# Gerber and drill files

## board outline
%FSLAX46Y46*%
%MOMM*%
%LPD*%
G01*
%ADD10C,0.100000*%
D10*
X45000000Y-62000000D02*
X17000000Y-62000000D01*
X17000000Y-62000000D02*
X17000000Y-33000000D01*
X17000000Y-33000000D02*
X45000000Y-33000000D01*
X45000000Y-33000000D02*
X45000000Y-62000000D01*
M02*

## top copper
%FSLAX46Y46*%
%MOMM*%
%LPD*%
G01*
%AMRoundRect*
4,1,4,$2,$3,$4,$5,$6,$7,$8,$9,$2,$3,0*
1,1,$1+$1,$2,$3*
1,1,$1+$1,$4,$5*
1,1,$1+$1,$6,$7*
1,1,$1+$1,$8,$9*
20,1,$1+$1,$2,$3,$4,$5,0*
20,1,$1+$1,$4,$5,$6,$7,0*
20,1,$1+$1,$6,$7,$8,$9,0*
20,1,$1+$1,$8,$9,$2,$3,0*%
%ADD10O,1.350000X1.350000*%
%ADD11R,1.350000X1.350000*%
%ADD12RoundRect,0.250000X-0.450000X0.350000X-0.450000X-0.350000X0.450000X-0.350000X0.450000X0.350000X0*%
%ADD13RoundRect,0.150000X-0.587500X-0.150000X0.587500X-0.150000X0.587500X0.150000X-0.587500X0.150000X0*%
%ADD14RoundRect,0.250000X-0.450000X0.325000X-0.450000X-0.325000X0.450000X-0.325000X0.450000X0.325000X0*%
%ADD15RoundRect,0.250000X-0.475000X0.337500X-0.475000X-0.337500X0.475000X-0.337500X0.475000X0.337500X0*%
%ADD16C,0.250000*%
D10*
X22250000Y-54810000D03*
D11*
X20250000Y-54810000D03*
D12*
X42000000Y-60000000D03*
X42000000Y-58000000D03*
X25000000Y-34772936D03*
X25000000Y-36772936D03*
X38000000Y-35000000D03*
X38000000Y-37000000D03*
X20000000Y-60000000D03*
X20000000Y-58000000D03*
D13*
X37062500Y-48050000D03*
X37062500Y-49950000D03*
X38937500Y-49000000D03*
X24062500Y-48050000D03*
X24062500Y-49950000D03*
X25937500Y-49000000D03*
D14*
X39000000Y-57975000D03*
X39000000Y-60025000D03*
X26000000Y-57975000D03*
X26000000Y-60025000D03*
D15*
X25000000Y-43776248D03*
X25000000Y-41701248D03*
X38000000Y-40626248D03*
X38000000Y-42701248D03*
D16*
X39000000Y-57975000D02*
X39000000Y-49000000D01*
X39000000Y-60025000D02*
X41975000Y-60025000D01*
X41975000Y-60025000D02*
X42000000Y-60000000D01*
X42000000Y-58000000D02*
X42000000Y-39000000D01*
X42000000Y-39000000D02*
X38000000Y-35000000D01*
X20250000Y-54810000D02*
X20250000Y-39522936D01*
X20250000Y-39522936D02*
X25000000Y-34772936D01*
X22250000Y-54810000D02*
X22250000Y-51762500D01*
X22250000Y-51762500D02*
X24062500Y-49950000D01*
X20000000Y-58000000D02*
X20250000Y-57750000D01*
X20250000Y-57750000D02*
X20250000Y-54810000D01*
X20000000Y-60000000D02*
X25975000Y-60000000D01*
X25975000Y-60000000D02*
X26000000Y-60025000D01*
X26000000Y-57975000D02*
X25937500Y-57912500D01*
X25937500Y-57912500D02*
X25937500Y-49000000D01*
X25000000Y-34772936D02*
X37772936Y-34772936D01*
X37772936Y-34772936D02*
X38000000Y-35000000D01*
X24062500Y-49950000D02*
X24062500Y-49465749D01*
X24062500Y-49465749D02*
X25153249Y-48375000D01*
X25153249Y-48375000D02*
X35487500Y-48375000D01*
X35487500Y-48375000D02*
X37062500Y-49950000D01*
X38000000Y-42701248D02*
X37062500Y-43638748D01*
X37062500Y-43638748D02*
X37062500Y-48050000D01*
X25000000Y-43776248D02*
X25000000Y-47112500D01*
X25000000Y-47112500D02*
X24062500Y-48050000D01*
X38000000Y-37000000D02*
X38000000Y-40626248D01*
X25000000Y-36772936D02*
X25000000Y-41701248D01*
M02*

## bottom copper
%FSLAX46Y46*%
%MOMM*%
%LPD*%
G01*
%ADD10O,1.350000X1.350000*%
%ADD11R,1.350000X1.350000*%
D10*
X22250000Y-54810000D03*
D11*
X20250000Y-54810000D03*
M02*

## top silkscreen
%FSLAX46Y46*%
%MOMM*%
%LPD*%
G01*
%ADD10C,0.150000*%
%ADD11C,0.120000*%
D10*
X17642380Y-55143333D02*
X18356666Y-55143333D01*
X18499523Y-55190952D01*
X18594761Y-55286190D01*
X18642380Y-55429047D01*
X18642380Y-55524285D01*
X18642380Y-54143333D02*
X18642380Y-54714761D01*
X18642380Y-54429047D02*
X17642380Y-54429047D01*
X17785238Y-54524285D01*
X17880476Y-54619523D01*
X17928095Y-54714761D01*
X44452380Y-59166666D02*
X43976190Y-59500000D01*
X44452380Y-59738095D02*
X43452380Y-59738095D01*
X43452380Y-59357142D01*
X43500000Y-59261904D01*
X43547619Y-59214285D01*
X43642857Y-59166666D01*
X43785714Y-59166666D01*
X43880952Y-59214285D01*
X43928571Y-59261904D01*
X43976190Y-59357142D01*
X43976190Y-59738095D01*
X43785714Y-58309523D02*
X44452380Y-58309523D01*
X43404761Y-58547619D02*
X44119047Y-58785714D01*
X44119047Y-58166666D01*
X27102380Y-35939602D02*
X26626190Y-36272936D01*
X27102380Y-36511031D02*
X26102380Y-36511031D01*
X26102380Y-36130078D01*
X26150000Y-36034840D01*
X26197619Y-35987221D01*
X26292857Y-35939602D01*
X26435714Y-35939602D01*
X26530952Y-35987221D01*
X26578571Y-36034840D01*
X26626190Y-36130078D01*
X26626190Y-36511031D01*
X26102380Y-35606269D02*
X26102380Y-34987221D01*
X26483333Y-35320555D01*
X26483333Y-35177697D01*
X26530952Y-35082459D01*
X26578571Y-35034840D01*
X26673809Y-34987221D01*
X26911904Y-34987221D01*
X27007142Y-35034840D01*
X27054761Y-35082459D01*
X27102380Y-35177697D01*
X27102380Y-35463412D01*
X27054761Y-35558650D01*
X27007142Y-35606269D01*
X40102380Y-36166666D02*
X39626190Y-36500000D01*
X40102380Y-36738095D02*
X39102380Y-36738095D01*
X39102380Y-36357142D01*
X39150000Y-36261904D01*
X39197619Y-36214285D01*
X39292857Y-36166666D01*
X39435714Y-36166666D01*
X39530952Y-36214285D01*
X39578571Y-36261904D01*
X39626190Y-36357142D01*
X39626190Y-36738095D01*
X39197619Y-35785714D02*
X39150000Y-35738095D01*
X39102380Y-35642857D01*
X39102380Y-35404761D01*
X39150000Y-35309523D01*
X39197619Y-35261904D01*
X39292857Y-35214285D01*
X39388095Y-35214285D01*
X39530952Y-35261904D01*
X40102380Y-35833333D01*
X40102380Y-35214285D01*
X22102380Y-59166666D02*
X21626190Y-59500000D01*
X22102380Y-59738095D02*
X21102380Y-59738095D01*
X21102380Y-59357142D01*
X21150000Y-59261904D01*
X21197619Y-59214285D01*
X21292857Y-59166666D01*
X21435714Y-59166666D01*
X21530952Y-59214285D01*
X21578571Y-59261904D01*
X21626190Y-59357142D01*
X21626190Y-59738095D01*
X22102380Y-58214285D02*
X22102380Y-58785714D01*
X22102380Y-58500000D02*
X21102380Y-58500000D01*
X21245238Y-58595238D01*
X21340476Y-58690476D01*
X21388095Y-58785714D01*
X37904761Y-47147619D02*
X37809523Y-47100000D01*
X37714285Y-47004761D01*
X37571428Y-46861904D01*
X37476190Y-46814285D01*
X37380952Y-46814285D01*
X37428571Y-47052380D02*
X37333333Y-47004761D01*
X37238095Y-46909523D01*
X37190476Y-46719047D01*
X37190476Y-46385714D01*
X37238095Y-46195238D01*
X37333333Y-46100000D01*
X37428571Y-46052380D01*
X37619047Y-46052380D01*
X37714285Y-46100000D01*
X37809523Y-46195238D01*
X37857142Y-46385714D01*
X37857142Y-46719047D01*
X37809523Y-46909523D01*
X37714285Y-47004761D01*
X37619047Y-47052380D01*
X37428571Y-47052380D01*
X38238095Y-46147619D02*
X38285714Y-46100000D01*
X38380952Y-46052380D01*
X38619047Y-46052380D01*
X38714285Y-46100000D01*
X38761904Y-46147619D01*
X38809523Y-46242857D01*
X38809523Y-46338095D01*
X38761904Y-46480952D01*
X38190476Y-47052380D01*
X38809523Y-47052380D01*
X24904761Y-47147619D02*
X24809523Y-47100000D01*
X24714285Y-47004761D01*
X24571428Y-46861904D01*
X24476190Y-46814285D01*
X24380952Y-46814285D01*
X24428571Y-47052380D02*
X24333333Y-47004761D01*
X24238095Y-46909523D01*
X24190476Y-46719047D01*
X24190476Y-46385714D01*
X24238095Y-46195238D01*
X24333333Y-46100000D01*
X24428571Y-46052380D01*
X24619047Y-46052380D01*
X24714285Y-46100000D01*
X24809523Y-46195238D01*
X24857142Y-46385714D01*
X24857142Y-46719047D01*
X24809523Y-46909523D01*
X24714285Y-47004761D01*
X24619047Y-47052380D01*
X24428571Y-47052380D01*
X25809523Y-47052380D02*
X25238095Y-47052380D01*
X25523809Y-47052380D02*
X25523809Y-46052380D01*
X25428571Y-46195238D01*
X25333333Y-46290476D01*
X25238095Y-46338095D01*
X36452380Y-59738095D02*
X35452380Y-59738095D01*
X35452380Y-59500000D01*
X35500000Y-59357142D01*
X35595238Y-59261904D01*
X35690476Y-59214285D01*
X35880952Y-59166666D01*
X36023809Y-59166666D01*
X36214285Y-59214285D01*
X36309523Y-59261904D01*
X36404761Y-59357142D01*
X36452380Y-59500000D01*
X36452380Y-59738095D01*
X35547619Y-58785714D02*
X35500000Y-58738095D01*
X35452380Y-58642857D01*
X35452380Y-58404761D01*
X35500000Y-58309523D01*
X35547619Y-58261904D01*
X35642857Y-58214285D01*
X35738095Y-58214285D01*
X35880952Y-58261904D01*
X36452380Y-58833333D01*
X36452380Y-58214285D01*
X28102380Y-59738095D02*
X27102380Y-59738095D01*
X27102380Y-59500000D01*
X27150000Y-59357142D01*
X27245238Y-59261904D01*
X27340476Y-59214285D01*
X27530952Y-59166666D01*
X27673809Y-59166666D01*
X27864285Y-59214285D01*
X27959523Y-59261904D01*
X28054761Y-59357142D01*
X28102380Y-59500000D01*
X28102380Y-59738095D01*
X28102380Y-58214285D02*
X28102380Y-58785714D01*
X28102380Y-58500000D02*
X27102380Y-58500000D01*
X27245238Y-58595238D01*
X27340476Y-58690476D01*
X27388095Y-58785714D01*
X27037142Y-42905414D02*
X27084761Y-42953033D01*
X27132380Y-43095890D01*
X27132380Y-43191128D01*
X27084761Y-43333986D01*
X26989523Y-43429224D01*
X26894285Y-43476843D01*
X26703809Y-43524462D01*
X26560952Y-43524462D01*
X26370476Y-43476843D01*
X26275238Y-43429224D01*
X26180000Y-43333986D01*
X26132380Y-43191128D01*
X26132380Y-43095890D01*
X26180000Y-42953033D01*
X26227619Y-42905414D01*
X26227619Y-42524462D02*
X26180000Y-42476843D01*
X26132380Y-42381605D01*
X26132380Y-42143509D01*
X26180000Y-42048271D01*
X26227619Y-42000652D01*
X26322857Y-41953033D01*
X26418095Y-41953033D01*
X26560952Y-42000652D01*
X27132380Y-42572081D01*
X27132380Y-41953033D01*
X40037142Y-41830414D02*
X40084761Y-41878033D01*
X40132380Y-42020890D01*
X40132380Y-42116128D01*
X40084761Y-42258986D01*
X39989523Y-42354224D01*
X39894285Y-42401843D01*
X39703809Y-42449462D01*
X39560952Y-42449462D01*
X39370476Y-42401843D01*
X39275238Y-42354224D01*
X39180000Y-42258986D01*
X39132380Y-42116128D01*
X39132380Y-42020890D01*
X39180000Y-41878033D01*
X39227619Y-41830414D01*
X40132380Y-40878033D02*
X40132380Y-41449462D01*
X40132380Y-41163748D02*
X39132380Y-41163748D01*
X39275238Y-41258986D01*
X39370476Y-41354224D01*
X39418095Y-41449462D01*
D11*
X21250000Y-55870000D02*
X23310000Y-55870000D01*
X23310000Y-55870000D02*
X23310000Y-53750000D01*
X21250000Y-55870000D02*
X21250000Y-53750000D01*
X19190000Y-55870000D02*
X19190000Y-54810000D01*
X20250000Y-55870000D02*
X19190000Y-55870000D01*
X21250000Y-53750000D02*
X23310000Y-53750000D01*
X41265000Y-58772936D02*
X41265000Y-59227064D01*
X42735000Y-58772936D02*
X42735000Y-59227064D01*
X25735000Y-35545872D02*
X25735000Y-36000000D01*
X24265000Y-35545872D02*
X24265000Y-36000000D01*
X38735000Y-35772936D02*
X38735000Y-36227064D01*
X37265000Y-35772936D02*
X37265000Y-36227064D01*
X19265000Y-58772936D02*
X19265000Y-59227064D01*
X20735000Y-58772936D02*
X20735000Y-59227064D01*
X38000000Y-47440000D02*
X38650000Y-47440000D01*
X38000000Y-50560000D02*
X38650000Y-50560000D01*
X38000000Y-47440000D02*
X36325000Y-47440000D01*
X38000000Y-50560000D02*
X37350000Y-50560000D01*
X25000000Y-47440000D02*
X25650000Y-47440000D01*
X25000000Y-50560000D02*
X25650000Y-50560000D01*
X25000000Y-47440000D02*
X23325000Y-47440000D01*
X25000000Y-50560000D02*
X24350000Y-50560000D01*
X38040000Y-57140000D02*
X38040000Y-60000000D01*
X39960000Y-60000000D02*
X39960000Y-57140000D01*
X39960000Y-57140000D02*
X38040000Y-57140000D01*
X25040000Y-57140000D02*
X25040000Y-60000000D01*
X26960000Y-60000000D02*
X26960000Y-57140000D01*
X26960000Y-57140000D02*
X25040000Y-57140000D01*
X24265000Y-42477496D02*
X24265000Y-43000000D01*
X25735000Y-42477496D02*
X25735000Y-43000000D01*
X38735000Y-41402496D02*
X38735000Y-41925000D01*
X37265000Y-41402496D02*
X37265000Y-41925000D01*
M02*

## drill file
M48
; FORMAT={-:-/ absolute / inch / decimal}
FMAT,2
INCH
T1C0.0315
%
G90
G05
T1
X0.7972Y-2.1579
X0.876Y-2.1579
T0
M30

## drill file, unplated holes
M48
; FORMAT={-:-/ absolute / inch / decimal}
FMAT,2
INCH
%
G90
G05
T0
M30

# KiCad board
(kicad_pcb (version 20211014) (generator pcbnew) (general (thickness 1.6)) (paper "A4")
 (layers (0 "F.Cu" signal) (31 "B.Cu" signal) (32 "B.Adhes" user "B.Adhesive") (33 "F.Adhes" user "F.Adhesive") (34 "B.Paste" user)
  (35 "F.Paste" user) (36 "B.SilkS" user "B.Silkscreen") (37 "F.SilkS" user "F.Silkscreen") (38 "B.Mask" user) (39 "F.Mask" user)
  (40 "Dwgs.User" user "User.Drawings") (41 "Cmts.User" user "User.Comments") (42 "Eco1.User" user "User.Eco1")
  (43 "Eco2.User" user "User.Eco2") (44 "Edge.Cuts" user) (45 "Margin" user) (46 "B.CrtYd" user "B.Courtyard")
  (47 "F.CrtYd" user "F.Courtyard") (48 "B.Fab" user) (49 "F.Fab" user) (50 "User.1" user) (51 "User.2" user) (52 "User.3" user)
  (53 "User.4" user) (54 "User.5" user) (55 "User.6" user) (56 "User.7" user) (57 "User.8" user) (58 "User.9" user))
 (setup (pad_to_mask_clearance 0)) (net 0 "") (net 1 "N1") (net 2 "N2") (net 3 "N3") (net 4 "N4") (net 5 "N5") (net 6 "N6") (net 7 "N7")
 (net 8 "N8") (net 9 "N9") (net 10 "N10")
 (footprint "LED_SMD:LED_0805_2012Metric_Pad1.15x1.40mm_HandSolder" (layer "F.Cu") (at 26 59 -90)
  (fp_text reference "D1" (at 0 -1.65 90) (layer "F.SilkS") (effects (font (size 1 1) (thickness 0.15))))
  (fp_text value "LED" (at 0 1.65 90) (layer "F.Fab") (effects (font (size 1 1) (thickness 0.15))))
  (fp_line (start 1 -0.96) (end -1.86 -0.96) (layer "F.SilkS") (width 0.12))
  (fp_line (start -1.86 -0.96) (end -1.86 0.96) (layer "F.SilkS") (width 0.12))
  (fp_line (start -1.86 0.96) (end 1 0.96) (layer "F.SilkS") (width 0.12))
  (pad "1" smd roundrect (at -1.025 0 270) (size 1.15 1.4) (layers "F.Cu" "F.Paste" "F.Mask") (roundrect_rratio 0.2173913043) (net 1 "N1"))
  (pad "2" smd roundrect (at 1.025 0 270) (size 1.15 1.4) (layers "F.Cu" "F.Paste" "F.Mask") (roundrect_rratio 0.2173913043) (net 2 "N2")))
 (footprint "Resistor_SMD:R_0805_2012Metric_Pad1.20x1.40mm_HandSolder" (layer "F.Cu") (at 25 35.772936 -90)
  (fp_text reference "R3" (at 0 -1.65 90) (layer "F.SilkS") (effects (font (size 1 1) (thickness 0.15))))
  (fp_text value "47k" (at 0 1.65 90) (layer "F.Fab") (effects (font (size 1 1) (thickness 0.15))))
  (fp_line (start -0.227064 0.735) (end 0.227064 0.735) (layer "F.SilkS") (width 0.12))
  (fp_line (start -0.227064 -0.735) (end 0.227064 -0.735) (layer "F.SilkS") (width 0.12))
  (pad "1" smd roundrect (at -1 0 270) (size 1.2 1.4) (layers "F.Cu" "F.Paste" "F.Mask") (roundrect_rratio 0.2083333333) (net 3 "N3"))
  (pad "2" smd roundrect (at 1 0 270) (size 1.2 1.4) (layers "F.Cu" "F.Paste" "F.Mask") (roundrect_rratio 0.2083333333) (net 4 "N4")))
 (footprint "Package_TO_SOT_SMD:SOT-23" (layer "F.Cu") (at 38 49)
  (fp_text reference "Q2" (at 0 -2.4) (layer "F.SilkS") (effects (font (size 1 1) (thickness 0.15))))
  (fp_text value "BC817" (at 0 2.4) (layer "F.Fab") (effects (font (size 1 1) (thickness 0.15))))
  (fp_line (start 0 -1.56) (end -1.675 -1.56) (layer "F.SilkS") (width 0.12))
  (fp_line (start 0 1.56) (end -0.65 1.56) (layer "F.SilkS") (width 0.12))
  (fp_line (start 0 1.56) (end 0.65 1.56) (layer "F.SilkS") (width 0.12))
  (fp_line (start 0 -1.56) (end 0.65 -1.56) (layer "F.SilkS") (width 0.12))
  (pad "1" smd roundrect (at -0.9375 -0.95) (size 1.475 0.6) (layers "F.Cu" "F.Paste" "F.Mask") (roundrect_rratio 0.25) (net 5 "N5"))
  (pad "2" smd roundrect (at -0.9375 0.95) (size 1.475 0.6) (layers "F.Cu" "F.Paste" "F.Mask") (roundrect_rratio 0.25) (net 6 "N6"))
  (pad "3" smd roundrect (at 0.9375 0) (size 1.475 0.6) (layers "F.Cu" "F.Paste" "F.Mask") (roundrect_rratio 0.25) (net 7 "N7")))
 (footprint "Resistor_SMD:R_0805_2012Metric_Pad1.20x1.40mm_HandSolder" (layer "F.Cu") (at 38 36 -90)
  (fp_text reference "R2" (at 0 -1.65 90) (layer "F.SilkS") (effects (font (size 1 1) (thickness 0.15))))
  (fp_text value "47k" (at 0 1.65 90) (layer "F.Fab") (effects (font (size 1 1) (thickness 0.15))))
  (fp_line (start -0.227064 -0.735) (end 0.227064 -0.735) (layer "F.SilkS") (width 0.12))
  (fp_line (start -0.227064 0.735) (end 0.227064 0.735) (layer "F.SilkS") (width 0.12))
  (pad "1" smd roundrect (at -1 0 270) (size 1.2 1.4) (layers "F.Cu" "F.Paste" "F.Mask") (roundrect_rratio 0.2083333333) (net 3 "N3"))
  (pad "2" smd roundrect (at 1 0 270) (size 1.2 1.4) (layers "F.Cu" "F.Paste" "F.Mask") (roundrect_rratio 0.2083333333) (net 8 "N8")))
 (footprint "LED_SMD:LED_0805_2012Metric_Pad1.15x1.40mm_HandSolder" (layer "F.Cu") (at 39 59 -90)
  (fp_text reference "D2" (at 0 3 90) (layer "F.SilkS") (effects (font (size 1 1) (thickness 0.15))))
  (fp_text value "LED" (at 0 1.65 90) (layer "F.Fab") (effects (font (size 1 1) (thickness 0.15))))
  (fp_line (start -1.86 -0.96) (end -1.86 0.96) (layer "F.SilkS") (width 0.12))
  (fp_line (start -1.86 0.96) (end 1 0.96) (layer "F.SilkS") (width 0.12))
  (fp_line (start 1 -0.96) (end -1.86 -0.96) (layer "F.SilkS") (width 0.12))
  (pad "1" smd roundrect (at -1.025 0 270) (size 1.15 1.4) (layers "F.Cu" "F.Paste" "F.Mask") (roundrect_rratio 0.2173913043) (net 7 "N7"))
  (pad "2" smd roundrect (at 1.025 0 270) (size 1.15 1.4) (layers "F.Cu" "F.Paste" "F.Mask") (roundrect_rratio 0.2173913043) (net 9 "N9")))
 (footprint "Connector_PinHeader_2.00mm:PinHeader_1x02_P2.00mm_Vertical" (layer "F.Cu") (at 20.25 54.81 90)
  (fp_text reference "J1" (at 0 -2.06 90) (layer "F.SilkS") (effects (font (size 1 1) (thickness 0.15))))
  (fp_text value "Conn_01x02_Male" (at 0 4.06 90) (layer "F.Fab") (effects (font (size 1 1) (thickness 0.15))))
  (fp_line (start -1.06 0) (end -1.06 -1.06) (layer "F.SilkS") (width 0.12))
  (fp_line (start -1.06 -1.06) (end 0 -1.06) (layer "F.SilkS") (width 0.12))
  (fp_line (start -1.06 1) (end 1.06 1) (layer "F.SilkS") (width 0.12))
  (fp_line (start -1.06 1) (end -1.06 3.06) (layer "F.SilkS") (width 0.12))
  (fp_line (start 1.06 1) (end 1.06 3.06) (layer "F.SilkS") (width 0.12))
  (fp_line (start -1.06 3.06) (end 1.06 3.06) (layer "F.SilkS") (width 0.12))
  (pad "1" thru_hole rect (at 0 0 90) (size 1.35 1.35) (drill 0.8) (layers *.Cu *.Mask) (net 3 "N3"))
  (pad "2" thru_hole oval (at 0 2 90) (size 1.35 1.35) (drill 0.8) (layers *.Cu *.Mask) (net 6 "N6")))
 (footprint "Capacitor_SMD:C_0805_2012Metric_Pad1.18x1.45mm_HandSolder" (layer "F.Cu") (at 38 41.663748 -90)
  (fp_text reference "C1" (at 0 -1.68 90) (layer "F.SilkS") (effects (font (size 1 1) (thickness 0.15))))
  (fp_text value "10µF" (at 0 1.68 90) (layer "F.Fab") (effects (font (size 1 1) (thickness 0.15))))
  (fp_line (start -0.261252 -0.735) (end 0.261252 -0.735) (layer "F.SilkS") (width 0.12))
  (fp_line (start -0.261252 0.735) (end 0.261252 0.735) (layer "F.SilkS") (width 0.12))
  (pad "1" smd roundrect (at -1.0375 0 270) (size 1.175 1.45) (layers "F.Cu" "F.Paste" "F.Mask") (roundrect_rratio 0.2127659574)
   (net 8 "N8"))
  (pad "2" smd roundrect (at 1.0375 0 270) (size 1.175 1.45) (layers "F.Cu" "F.Paste" "F.Mask") (roundrect_rratio 0.2127659574) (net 5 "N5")))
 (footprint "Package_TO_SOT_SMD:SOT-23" (layer "F.Cu") (at 25 49)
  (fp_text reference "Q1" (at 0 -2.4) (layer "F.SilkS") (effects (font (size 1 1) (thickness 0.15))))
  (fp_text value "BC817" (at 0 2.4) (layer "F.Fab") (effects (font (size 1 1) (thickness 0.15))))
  (fp_line (start 0 -1.56) (end -1.675 -1.56) (layer "F.SilkS") (width 0.12))
  (fp_line (start 0 -1.56) (end 0.65 -1.56) (layer "F.SilkS") (width 0.12))
  (fp_line (start 0 1.56) (end -0.65 1.56) (layer "F.SilkS") (width 0.12))
  (fp_line (start 0 1.56) (end 0.65 1.56) (layer "F.SilkS") (width 0.12))
  (pad "1" smd roundrect (at -0.9375 -0.95) (size 1.475 0.6) (layers "F.Cu" "F.Paste" "F.Mask") (roundrect_rratio 0.25) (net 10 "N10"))
  (pad "2" smd roundrect (at -0.9375 0.95) (size 1.475 0.6) (layers "F.Cu" "F.Paste" "F.Mask") (roundrect_rratio 0.25) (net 6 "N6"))
  (pad "3" smd roundrect (at 0.9375 0) (size 1.475 0.6) (layers "F.Cu" "F.Paste" "F.Mask") (roundrect_rratio 0.25) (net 1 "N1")))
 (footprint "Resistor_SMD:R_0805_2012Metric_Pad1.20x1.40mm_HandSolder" (layer "F.Cu") (at 42 59 -90)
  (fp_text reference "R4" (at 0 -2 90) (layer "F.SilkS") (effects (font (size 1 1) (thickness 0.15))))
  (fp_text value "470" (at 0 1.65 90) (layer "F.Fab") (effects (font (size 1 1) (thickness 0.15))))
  (fp_line (start -0.227064 -0.735) (end 0.227064 -0.735) (layer "F.SilkS") (width 0.12))
  (fp_line (start -0.227064 0.735) (end 0.227064 0.735) (layer "F.SilkS") (width 0.12))
  (pad "1" smd roundrect (at -1 0 270) (size 1.2 1.4) (layers "F.Cu" "F.Paste" "F.Mask") (roundrect_rratio 0.2083333333) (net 3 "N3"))
  (pad "2" smd roundrect (at 1 0 270) (size 1.2 1.4) (layers "F.Cu" "F.Paste" "F.Mask") (roundrect_rratio 0.2083333333) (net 9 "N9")))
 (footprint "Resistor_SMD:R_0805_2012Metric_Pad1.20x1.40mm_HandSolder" (layer "F.Cu") (at 20 59 -90)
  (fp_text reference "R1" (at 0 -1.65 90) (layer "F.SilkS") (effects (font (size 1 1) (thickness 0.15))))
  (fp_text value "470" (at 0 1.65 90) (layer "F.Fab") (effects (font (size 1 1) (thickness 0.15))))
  (fp_line (start -0.227064 0.735) (end 0.227064 0.735) (layer "F.SilkS") (width 0.12))
  (fp_line (start -0.227064 -0.735) (end 0.227064 -0.735) (layer "F.SilkS") (width 0.12))
  (pad "1" smd roundrect (at -1 0 270) (size 1.2 1.4) (layers "F.Cu" "F.Paste" "F.Mask") (roundrect_rratio 0.2083333333) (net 3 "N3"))
  (pad "2" smd roundrect (at 1 0 270) (size 1.2 1.4) (layers "F.Cu" "F.Paste" "F.Mask") (roundrect_rratio 0.2083333333) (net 2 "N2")))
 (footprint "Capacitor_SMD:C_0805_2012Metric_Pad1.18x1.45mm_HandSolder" (layer "F.Cu") (at 25 42.738748 -90)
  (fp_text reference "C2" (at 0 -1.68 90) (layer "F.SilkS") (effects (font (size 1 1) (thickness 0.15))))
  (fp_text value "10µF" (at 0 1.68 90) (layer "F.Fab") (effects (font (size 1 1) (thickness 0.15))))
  (fp_line (start -0.261252 -0.735) (end 0.261252 -0.735) (layer "F.SilkS") (width 0.12))
  (fp_line (start -0.261252 0.735) (end 0.261252 0.735) (layer "F.SilkS") (width 0.12))
  (pad "1" smd roundrect (at -1.0375 0 270) (size 1.175 1.45) (layers "F.Cu" "F.Paste" "F.Mask") (roundrect_rratio 0.2127659574)
   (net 4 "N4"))
  (pad "2" smd roundrect (at 1.0375 0 270) (size 1.175 1.45) (layers "F.Cu" "F.Paste" "F.Mask") (roundrect_rratio 0.2127659574)
   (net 10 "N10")))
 (gr_rect (start 45 62) (end 17 33) (layer "Edge.Cuts") (width 0.1) (fill none))
 (segment (start 38 37) (end 38 40.626248) (width 0.25) (layer "F.Cu") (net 8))
 (segment (start 37.0625 43.638748) (end 37.0625 48.05) (width 0.25) (layer "F.Cu") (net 5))
 (segment (start 38 42.701248) (end 37.0625 43.638748) (width 0.25) (layer "F.Cu") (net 5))
 (segment (start 25 36.772936) (end 25 41.701248) (width 0.25) (layer "F.Cu") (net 4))
 (segment (start 25 47.1125) (end 24.0625 48.05) (width 0.25) (layer "F.Cu") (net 10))
 (segment (start 25 43.776248) (end 25 47.1125) (width 0.25) (layer "F.Cu") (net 10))
 (segment (start 26 57.975) (end 25.9375 57.9125) (width 0.25) (layer "F.Cu") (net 1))
 (segment (start 25.9375 57.9125) (end 25.9375 49) (width 0.25) (layer "F.Cu") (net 1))
 (segment (start 25.975 60) (end 26 60.025) (width 0.25) (layer "F.Cu") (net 2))
 (segment (start 20 60) (end 25.975 60) (width 0.25) (layer "F.Cu") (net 2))
 (segment (start 39 57.975) (end 39 49) (width 0.25) (layer "F.Cu") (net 7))
 (segment (start 41.975 60.025) (end 42 60) (width 0.25) (layer "F.Cu") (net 9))
 (segment (start 39 60.025) (end 41.975 60.025) (width 0.25) (layer "F.Cu") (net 9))
 (segment (start 25.153249 48.375) (end 35.4875 48.375) (width 0.25) (layer "F.Cu") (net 6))
 (segment (start 22.25 54.81) (end 22.25 51.7625) (width 0.25) (layer "F.Cu") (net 6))
 (segment (start 22.25 51.7625) (end 24.0625 49.95) (width 0.25) (layer "F.Cu") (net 6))
 (segment (start 35.4875 48.375) (end 37.0625 49.95) (width 0.25) (layer "F.Cu") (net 6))
 (segment (start 24.0625 49.95) (end 24.0625 49.465749) (width 0.25) (layer "F.Cu") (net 6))
 (segment (start 24.0625 49.465749) (end 25.153249 48.375) (width 0.25) (layer "F.Cu") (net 6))
 (segment (start 42 58) (end 42 39) (width 0.25) (layer "F.Cu") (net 3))
 (segment (start 25 34.772936) (end 37.772936 34.772936) (width 0.25) (layer "F.Cu") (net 3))
 (segment (start 20.25 57.75) (end 20.25 54.81) (width 0.25) (layer "F.Cu") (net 3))
 (segment (start 20.25 39.522936) (end 25 34.772936) (width 0.25) (layer "F.Cu") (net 3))
 (segment (start 20 58) (end 20.25 57.75) (width 0.25) (layer "F.Cu") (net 3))
 (segment (start 42 39) (end 38 35) (width 0.25) (layer "F.Cu") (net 3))
 (segment (start 20.25 54.81) (end 20.25 39.522936) (width 0.25) (layer "F.Cu") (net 3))
 (segment (start 37.772936 34.772936) (end 38 35) (width 0.25) (layer "F.Cu") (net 3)))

